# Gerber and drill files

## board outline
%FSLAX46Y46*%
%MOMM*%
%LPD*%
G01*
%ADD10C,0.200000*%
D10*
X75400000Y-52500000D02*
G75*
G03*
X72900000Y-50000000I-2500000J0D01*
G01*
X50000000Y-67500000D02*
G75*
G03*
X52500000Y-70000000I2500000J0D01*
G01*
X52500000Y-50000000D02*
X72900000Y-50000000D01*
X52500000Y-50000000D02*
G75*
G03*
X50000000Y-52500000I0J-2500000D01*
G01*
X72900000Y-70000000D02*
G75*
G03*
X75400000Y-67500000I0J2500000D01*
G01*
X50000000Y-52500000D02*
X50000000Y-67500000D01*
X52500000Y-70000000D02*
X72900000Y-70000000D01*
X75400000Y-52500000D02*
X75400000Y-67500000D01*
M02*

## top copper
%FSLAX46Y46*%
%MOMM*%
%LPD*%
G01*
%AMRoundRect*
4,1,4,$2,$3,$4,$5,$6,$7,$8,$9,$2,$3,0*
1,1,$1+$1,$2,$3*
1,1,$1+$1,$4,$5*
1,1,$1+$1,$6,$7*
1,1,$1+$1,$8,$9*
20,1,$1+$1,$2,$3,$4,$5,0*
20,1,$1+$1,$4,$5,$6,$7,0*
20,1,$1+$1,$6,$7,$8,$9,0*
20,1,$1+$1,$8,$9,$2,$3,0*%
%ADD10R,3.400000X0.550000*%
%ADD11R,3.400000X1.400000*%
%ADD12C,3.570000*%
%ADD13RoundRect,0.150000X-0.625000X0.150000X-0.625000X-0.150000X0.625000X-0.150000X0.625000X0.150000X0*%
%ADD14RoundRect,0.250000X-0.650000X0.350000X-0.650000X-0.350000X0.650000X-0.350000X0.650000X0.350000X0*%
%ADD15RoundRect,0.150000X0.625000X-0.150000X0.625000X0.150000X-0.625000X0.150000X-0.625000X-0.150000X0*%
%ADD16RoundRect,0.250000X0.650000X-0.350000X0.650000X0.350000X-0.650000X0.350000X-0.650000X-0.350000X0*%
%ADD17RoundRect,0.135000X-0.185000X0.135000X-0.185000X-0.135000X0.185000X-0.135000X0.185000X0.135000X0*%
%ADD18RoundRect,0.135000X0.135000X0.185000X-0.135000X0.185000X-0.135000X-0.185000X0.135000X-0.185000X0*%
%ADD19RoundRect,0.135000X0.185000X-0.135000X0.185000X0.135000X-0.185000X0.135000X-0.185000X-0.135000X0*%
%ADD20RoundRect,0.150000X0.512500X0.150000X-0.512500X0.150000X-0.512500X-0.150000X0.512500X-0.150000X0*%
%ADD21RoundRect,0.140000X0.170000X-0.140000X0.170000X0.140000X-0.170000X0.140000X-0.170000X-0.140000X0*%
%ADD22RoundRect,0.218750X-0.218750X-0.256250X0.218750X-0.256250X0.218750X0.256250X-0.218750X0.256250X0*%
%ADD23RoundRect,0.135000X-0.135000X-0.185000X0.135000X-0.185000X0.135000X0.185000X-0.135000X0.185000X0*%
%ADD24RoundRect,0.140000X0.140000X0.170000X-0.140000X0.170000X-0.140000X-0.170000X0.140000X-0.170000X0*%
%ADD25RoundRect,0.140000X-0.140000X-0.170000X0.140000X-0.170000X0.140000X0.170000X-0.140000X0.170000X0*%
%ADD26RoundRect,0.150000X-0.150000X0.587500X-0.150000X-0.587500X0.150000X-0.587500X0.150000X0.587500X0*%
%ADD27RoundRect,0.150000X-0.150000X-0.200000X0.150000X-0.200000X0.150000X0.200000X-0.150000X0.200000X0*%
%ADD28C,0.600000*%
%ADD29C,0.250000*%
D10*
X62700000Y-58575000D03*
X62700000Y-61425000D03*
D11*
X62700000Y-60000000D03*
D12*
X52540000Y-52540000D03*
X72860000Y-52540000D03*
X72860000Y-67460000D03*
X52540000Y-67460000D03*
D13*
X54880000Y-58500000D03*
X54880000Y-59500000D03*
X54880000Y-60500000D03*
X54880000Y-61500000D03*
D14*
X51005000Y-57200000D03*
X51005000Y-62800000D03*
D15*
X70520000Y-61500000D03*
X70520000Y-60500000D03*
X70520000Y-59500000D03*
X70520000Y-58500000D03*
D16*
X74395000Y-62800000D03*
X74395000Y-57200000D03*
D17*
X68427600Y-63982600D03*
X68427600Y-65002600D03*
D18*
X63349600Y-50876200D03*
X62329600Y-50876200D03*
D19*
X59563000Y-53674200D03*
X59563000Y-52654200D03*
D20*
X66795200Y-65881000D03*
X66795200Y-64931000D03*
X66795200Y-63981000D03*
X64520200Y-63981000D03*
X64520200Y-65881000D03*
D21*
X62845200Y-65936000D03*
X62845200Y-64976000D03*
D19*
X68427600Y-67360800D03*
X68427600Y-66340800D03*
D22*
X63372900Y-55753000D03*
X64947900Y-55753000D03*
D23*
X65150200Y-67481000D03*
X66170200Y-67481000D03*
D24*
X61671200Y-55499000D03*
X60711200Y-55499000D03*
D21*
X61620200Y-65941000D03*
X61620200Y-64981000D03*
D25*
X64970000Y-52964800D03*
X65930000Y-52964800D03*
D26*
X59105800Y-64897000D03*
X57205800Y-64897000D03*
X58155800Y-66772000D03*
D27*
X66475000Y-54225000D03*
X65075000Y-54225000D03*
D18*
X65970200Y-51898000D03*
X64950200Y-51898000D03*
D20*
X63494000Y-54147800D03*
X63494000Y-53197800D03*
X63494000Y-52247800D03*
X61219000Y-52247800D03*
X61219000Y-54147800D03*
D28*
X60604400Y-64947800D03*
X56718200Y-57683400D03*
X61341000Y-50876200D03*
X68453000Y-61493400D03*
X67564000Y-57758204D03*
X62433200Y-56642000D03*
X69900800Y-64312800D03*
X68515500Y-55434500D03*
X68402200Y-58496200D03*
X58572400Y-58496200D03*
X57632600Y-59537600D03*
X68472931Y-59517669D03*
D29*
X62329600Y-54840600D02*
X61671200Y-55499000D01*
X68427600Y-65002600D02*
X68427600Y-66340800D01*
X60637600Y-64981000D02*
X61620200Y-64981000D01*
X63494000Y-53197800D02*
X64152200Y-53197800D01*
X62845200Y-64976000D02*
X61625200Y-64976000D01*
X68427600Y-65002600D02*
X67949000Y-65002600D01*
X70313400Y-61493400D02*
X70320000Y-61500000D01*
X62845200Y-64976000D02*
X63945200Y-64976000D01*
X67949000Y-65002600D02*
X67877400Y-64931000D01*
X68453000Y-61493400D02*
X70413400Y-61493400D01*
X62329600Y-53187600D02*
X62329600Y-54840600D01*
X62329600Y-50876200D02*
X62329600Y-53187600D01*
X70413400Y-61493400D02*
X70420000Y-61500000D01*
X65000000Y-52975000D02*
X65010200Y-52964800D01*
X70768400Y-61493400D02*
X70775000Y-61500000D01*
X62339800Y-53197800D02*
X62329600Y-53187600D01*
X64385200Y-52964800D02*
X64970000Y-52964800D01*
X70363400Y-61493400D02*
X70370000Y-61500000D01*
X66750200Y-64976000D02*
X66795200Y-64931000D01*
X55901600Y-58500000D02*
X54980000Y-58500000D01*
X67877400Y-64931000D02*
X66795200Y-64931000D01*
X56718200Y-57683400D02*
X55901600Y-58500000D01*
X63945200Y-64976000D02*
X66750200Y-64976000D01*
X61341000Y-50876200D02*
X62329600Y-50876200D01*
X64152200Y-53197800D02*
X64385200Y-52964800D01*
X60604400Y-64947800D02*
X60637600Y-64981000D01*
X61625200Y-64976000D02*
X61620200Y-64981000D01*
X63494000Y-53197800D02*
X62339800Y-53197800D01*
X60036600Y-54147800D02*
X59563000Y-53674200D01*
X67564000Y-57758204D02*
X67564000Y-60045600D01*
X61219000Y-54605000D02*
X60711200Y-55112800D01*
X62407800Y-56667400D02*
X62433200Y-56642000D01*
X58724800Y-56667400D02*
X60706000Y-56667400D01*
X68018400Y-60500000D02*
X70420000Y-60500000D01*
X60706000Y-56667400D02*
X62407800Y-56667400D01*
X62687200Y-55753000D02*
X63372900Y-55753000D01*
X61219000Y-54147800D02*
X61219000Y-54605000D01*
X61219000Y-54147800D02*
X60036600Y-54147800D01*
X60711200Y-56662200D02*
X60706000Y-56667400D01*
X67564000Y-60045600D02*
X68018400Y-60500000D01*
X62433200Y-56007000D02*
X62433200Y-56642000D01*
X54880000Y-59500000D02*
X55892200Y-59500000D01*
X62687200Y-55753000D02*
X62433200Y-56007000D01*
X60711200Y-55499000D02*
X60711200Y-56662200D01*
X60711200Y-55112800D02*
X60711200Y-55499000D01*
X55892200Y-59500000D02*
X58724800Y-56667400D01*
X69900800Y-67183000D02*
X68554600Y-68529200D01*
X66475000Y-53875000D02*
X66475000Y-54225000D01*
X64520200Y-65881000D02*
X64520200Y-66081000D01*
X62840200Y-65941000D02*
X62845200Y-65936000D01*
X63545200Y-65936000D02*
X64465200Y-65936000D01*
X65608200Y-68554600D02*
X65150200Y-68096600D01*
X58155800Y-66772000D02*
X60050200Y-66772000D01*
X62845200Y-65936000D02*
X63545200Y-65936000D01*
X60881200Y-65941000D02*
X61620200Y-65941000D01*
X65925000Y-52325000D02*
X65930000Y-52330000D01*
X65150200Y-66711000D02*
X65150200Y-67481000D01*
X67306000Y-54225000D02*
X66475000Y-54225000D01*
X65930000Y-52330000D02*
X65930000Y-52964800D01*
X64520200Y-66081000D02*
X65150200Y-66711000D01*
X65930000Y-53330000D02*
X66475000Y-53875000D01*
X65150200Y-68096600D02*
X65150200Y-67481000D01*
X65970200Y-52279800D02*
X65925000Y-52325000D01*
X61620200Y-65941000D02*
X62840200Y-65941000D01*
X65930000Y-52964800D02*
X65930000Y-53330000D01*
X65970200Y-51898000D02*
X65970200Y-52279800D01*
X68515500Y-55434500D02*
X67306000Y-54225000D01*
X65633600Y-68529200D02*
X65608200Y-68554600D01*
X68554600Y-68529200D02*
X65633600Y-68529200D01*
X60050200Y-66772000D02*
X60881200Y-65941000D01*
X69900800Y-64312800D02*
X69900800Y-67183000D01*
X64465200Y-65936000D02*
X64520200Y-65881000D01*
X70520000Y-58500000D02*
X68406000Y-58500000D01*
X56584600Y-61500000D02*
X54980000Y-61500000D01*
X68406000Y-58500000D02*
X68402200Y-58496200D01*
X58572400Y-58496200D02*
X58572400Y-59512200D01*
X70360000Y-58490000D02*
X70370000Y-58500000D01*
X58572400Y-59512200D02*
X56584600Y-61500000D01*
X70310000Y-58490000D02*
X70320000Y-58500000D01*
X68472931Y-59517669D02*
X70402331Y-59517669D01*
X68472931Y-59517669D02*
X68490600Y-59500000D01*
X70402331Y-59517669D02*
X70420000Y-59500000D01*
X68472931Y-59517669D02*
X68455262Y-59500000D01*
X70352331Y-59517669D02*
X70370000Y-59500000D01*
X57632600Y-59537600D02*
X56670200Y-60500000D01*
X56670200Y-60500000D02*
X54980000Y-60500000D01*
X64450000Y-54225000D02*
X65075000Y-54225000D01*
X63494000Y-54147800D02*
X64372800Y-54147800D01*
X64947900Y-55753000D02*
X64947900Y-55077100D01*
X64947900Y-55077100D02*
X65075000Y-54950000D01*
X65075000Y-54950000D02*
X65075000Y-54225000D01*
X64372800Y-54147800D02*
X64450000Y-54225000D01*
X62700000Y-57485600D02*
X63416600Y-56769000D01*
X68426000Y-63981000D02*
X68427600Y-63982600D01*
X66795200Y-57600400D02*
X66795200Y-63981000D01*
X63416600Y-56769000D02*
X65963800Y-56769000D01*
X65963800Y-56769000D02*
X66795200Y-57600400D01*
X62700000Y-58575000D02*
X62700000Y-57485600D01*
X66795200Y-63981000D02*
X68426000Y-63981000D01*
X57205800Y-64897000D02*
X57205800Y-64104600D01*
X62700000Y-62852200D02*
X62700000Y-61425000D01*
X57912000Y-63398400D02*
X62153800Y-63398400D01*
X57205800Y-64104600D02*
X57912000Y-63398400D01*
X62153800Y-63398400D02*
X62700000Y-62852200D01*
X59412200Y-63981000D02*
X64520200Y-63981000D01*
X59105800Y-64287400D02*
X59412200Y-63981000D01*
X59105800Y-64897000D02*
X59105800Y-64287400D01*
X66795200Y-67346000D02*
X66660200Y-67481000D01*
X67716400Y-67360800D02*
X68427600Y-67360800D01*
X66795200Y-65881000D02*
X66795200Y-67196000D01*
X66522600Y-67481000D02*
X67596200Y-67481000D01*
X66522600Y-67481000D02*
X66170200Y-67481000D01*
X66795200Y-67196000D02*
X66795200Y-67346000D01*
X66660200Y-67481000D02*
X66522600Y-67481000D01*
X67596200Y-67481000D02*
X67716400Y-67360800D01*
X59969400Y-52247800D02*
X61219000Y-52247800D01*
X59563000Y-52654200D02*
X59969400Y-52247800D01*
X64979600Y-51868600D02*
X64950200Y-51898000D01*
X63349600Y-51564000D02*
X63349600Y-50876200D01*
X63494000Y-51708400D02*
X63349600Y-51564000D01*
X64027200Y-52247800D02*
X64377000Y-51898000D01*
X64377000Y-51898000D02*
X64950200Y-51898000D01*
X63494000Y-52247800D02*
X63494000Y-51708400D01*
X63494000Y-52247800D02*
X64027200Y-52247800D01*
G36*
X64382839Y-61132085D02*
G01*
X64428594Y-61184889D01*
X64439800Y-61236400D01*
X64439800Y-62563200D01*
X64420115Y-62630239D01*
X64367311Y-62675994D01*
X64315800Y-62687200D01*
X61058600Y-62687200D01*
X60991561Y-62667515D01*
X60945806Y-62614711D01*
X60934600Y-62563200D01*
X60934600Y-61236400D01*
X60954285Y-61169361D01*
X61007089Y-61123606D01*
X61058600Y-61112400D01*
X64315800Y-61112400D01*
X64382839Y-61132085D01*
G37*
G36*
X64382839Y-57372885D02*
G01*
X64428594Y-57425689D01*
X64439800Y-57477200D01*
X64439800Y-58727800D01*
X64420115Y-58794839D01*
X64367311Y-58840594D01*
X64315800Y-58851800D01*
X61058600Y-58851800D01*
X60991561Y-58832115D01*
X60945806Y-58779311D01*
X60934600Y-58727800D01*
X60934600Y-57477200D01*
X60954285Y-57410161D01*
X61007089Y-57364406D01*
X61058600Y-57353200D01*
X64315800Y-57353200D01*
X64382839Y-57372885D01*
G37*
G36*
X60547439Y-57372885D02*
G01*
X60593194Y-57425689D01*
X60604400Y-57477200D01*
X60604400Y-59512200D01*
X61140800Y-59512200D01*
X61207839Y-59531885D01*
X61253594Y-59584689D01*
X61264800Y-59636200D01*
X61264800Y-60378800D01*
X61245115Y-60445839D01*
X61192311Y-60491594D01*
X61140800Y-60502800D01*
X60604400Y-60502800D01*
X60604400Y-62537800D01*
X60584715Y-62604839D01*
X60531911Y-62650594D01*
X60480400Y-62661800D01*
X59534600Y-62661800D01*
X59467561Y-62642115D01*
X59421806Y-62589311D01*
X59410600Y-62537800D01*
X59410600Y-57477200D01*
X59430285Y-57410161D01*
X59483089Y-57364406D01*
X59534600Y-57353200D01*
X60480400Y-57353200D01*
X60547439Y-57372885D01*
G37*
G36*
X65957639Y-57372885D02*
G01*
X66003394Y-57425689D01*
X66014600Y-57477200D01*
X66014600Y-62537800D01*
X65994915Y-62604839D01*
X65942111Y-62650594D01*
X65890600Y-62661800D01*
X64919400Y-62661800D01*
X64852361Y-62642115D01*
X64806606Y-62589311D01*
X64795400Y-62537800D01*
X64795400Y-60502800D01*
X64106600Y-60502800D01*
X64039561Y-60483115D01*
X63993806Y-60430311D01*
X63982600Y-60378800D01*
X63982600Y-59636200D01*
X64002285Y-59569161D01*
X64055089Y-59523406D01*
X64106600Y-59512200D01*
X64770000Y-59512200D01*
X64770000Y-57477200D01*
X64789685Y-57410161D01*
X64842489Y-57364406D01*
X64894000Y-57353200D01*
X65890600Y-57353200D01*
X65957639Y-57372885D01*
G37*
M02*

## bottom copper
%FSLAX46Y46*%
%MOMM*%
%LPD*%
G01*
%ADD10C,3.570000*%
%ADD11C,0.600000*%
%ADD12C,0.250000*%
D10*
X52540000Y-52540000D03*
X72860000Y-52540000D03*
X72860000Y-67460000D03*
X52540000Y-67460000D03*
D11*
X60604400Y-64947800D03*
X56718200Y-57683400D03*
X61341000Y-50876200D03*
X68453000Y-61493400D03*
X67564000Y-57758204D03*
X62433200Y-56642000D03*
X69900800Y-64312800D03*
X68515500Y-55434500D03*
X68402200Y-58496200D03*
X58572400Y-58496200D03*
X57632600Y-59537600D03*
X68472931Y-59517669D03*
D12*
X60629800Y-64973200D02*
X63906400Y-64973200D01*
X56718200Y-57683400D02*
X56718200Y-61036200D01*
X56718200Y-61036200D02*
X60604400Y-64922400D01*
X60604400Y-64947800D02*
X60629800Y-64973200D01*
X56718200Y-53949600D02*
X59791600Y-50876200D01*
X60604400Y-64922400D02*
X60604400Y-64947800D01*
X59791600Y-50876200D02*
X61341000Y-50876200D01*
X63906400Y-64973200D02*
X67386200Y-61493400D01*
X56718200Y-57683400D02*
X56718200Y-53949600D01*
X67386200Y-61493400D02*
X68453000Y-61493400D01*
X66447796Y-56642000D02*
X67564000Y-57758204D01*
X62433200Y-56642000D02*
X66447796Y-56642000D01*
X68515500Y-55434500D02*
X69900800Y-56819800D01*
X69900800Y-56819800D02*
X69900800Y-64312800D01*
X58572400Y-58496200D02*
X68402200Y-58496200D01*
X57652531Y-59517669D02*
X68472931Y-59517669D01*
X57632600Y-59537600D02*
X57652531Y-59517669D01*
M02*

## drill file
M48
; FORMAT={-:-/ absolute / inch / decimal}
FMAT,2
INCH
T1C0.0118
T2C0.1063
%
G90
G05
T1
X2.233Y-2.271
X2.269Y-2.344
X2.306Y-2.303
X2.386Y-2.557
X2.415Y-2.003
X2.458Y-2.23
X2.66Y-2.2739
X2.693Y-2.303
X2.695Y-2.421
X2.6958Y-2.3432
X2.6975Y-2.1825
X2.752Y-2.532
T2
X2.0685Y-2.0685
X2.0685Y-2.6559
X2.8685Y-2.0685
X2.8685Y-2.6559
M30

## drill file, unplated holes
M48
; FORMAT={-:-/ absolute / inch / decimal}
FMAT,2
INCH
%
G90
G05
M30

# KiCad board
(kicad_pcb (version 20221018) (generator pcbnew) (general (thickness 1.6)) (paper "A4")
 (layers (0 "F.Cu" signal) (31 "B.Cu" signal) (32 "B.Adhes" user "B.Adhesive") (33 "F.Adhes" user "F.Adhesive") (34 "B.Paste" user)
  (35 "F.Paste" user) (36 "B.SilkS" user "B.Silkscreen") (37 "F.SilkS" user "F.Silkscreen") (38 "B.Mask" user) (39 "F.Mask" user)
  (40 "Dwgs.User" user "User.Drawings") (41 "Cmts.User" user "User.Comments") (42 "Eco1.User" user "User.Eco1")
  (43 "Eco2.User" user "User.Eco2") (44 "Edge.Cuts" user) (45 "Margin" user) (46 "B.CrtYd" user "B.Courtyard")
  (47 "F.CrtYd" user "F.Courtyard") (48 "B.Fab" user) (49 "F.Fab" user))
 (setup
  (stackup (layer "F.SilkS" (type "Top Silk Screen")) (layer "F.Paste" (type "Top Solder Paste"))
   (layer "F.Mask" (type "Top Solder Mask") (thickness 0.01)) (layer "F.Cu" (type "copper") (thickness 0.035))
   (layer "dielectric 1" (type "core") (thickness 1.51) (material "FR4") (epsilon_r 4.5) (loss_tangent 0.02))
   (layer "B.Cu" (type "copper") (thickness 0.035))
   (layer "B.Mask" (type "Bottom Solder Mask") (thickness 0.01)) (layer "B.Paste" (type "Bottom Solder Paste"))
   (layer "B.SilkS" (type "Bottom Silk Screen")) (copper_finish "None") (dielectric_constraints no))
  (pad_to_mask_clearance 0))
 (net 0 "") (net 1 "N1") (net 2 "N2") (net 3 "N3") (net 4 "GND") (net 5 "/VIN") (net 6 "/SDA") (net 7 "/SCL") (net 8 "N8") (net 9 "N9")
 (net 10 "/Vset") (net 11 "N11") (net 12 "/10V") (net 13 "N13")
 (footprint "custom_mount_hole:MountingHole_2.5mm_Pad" (layer "F.Cu") (at 52.54 52.54)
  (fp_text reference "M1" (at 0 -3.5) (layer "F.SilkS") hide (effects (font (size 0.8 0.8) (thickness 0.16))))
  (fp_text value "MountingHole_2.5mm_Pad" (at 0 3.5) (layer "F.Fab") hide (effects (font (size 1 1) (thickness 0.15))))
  (pad "~" thru_hole circle (at 0 0) (size 3.57 3.57) (drill 2.7) (layers "*.Cu" "*.Mask")))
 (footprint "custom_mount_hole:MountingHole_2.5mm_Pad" (layer "F.Cu") (at 72.86 52.54)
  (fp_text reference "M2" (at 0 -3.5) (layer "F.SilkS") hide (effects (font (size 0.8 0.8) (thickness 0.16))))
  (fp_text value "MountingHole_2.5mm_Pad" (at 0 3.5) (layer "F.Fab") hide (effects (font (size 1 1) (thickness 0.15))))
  (pad "~" thru_hole circle (at 0 0) (size 3.57 3.57) (drill 2.7) (layers "*.Cu" "*.Mask")))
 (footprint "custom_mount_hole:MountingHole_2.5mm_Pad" (layer "F.Cu") (at 72.86 67.46)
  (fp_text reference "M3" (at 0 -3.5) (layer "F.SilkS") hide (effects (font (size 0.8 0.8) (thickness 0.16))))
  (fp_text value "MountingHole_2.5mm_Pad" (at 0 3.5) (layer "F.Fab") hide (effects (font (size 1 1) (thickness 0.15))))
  (pad "~" thru_hole circle (at 0 0) (size 3.57 3.57) (drill 2.7) (layers "*.Cu" "*.Mask")))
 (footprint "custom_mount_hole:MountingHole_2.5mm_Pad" (layer "F.Cu") (at 52.54 67.46)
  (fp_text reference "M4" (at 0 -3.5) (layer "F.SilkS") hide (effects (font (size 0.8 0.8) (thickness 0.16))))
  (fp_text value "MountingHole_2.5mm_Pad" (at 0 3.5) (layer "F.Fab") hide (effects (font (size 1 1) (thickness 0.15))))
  (pad "~" thru_hole circle (at 0 0) (size 3.57 3.57) (drill 2.7) (layers "*.Cu" "*.Mask")))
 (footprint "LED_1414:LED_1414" (layer "F.Cu") (at 62.7 60 -90)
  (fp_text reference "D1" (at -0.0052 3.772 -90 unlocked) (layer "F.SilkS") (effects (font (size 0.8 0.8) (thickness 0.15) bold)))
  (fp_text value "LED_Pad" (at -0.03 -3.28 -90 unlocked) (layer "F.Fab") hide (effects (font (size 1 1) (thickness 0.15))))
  (pad "1" smd rect (at -1.425 0 270) (size 0.55 3.4) (layers "F.Cu" "F.Paste" "F.Mask") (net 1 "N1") (thermal_bridge_angle 45))
  (pad "2" smd rect (at 1.425 0 270) (size 0.55 3.4) (layers "F.Cu" "F.Paste" "F.Mask") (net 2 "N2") (thermal_bridge_angle 45))
  (pad "3" smd rect (at 0 0 270) (size 1.4 3.4) (layers "F.Cu" "F.Paste" "F.Mask") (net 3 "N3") (thermal_bridge_angle 45)))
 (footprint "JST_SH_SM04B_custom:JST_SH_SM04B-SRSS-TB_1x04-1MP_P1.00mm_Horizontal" (layer "F.Cu") (at 52.88 60 -90)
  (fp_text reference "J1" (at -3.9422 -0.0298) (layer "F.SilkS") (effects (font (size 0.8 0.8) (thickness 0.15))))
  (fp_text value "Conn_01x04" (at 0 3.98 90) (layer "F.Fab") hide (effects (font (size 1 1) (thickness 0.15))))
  (pad "1" smd roundrect (at -1.5 -2 270) (size 0.6 1.55) (layers "F.Cu" "F.Paste" "F.Mask") (roundrect_rratio 0.25) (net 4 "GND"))
  (pad "2" smd roundrect (at -0.5 -2 270) (size 0.6 1.55) (layers "F.Cu" "F.Paste" "F.Mask") (roundrect_rratio 0.25) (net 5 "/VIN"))
  (pad "3" smd roundrect (at 0.5 -2 270) (size 0.6 1.55) (layers "F.Cu" "F.Paste" "F.Mask") (roundrect_rratio 0.25) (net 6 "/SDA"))
  (pad "4" smd roundrect (at 1.5 -2 270) (size 0.6 1.55) (layers "F.Cu" "F.Paste" "F.Mask") (roundrect_rratio 0.25) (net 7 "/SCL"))
  (pad "MP" smd roundrect (at -2.8 1.875 270) (size 1.2 1.8) (layers "F.Cu" "F.Paste" "F.Mask") (roundrect_rratio 0.2083333333))
  (pad "MP" smd roundrect (at 2.8 1.875 270) (size 1.2 1.8) (layers "F.Cu" "F.Paste" "F.Mask") (roundrect_rratio 0.2083333333)))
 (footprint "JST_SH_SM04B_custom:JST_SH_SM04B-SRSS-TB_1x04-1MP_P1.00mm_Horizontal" (layer "F.Cu") (at 72.52 60 90)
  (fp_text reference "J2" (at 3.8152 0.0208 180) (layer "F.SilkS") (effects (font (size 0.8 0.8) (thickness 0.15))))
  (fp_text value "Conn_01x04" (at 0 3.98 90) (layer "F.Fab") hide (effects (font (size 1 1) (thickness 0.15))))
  (pad "1" smd roundrect (at -1.5 -2 90) (size 0.6 1.55) (layers "F.Cu" "F.Paste" "F.Mask") (roundrect_rratio 0.25) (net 4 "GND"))
  (pad "2" smd roundrect (at -0.5 -2 90) (size 0.6 1.55) (layers "F.Cu" "F.Paste" "F.Mask") (roundrect_rratio 0.25) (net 5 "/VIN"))
  (pad "3" smd roundrect (at 0.5 -2 90) (size 0.6 1.55) (layers "F.Cu" "F.Paste" "F.Mask") (roundrect_rratio 0.25) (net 6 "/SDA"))
  (pad "4" smd roundrect (at 1.5 -2 90) (size 0.6 1.55) (layers "F.Cu" "F.Paste" "F.Mask") (roundrect_rratio 0.25) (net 7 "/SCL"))
  (pad "MP" smd roundrect (at -2.8 1.875 90) (size 1.2 1.8) (layers "F.Cu" "F.Paste" "F.Mask") (roundrect_rratio 0.2083333333))
  (pad "MP" smd roundrect (at 2.8 1.875 90) (size 1.2 1.8) (layers "F.Cu" "F.Paste" "F.Mask") (roundrect_rratio 0.2083333333)))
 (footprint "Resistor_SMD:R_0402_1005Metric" (layer "F.Cu") (at 68.4276 64.4926 -90)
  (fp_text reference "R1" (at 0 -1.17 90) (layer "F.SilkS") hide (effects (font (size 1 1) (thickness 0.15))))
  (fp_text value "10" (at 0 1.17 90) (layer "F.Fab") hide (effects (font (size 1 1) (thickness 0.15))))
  (pad "1" smd roundrect (at -0.51 0 270) (size 0.54 0.64) (layers "F.Cu" "F.Paste" "F.Mask") (roundrect_rratio 0.25) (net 1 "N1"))
  (pad "2" smd roundrect (at 0.51 0 270) (size 0.54 0.64) (layers "F.Cu" "F.Paste" "F.Mask") (roundrect_rratio 0.25) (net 4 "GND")))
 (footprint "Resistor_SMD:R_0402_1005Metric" (layer "F.Cu") (at 62.8396 50.8762 180)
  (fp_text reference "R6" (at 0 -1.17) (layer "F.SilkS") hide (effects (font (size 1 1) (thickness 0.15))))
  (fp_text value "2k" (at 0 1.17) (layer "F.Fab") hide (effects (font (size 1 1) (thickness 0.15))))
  (pad "1" smd roundrect (at -0.51 0 180) (size 0.54 0.64) (layers "F.Cu" "F.Paste" "F.Mask") (roundrect_rratio 0.25) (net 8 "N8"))
  (pad "2" smd roundrect (at 0.51 0 180) (size 0.54 0.64) (layers "F.Cu" "F.Paste" "F.Mask") (roundrect_rratio 0.25) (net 4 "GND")))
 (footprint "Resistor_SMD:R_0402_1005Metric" (layer "F.Cu") (at 59.563 53.1642 90)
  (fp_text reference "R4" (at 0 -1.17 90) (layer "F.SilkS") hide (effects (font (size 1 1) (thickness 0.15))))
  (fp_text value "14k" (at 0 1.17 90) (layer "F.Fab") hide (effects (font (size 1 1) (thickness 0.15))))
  (pad "1" smd roundrect (at -0.51 0 90) (size 0.54 0.64) (layers "F.Cu" "F.Paste" "F.Mask") (roundrect_rratio 0.25) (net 5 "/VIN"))
  (pad "2" smd roundrect (at 0.51 0 90) (size 0.54 0.64) (layers "F.Cu" "F.Paste" "F.Mask") (roundrect_rratio 0.25) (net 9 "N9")))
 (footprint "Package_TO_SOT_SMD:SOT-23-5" (layer "F.Cu") (at 65.6577 64.931 180)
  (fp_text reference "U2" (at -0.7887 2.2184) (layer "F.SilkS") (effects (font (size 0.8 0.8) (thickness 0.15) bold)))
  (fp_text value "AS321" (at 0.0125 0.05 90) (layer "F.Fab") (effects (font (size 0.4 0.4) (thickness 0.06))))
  (pad "1" smd roundrect (at -1.1375 -0.95 180) (size 1.325 0.6) (layers "F.Cu" "F.Paste" "F.Mask") (roundrect_rratio 0.25) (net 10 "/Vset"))
  (pad "2" smd roundrect (at -1.1375 0 180) (size 1.325 0.6) (layers "F.Cu" "F.Paste" "F.Mask") (roundrect_rratio 0.25) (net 4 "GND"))
  (pad "3" smd roundrect (at -1.1375 0.95 180) (size 1.325 0.6) (layers "F.Cu" "F.Paste" "F.Mask") (roundrect_rratio 0.25) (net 1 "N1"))
  (pad "4" smd roundrect (at 1.1375 0.95 180) (size 1.325 0.6) (layers "F.Cu" "F.Paste" "F.Mask") (roundrect_rratio 0.25) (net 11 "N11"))
  (pad "5" smd roundrect (at 1.1375 -0.95 180) (size 1.325 0.6) (layers "F.Cu" "F.Paste" "F.Mask") (roundrect_rratio 0.25) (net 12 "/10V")))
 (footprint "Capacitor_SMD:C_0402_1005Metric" (layer "F.Cu") (at 62.8452 65.456 90)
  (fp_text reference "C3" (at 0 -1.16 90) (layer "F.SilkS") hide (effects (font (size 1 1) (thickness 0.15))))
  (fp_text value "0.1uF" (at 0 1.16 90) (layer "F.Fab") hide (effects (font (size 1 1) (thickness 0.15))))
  (pad "1" smd roundrect (at -0.48 0 90) (size 0.56 0.62) (layers "F.Cu" "F.Paste" "F.Mask") (roundrect_rratio 0.25) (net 12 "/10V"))
  (pad "2" smd roundrect (at 0.48 0 90) (size 0.56 0.62) (layers "F.Cu" "F.Paste" "F.Mask") (roundrect_rratio 0.25) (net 4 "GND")))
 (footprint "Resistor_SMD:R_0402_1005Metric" (layer "F.Cu") (at 68.4276 66.8508 90)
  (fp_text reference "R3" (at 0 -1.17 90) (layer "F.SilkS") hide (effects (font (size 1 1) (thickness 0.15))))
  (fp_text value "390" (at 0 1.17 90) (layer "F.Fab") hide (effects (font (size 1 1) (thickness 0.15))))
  (pad "1" smd roundrect (at -0.51 0 90) (size 0.54 0.64) (layers "F.Cu" "F.Paste" "F.Mask") (roundrect_rratio 0.25) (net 10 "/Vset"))
  (pad "2" smd roundrect (at 0.51 0 90) (size 0.54 0.64) (layers "F.Cu" "F.Paste" "F.Mask") (roundrect_rratio 0.25) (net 4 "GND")))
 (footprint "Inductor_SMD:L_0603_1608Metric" (layer "F.Cu") (at 64.1604 55.753)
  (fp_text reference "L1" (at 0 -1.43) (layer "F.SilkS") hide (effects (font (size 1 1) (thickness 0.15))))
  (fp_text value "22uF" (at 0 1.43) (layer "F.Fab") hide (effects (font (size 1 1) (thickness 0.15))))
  (pad "1" smd roundrect (at -0.7875 0) (size 0.875 0.95) (layers "F.Cu" "F.Paste" "F.Mask") (roundrect_rratio 0.25) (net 5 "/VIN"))
  (pad "2" smd roundrect (at 0.7875 0) (size 0.875 0.95) (layers "F.Cu" "F.Paste" "F.Mask") (roundrect_rratio 0.25) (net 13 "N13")))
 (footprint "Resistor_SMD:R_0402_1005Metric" (layer "F.Cu") (at 65.6602 67.481)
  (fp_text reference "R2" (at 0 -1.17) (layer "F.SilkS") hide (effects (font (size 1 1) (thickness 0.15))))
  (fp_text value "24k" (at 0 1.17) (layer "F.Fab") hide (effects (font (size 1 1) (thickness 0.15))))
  (pad "1" smd roundrect (at -0.51 0) (size 0.54 0.64) (layers "F.Cu" "F.Paste" "F.Mask") (roundrect_rratio 0.25) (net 12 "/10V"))
  (pad "2" smd roundrect (at 0.51 0) (size 0.54 0.64) (layers "F.Cu" "F.Paste" "F.Mask") (roundrect_rratio 0.25) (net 10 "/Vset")))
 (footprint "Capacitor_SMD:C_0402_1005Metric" (layer "F.Cu") (at 61.1912 55.499 180)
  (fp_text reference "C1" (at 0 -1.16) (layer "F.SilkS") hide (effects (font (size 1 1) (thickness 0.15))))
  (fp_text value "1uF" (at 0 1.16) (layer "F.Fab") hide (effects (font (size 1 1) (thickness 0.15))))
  (pad "1" smd roundrect (at -0.48 0 180) (size 0.56 0.62) (layers "F.Cu" "F.Paste" "F.Mask") (roundrect_rratio 0.25) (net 4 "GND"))
  (pad "2" smd roundrect (at 0.48 0 180) (size 0.56 0.62) (layers "F.Cu" "F.Paste" "F.Mask") (roundrect_rratio 0.25) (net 5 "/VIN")))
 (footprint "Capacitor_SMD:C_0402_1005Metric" (layer "F.Cu") (at 61.6202 65.461 90)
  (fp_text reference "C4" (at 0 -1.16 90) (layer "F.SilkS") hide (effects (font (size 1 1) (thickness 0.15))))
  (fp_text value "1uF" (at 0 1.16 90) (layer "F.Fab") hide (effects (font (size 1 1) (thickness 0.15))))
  (pad "1" smd roundrect (at -0.48 0 90) (size 0.56 0.62) (layers "F.Cu" "F.Paste" "F.Mask") (roundrect_rratio 0.25) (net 12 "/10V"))
  (pad "2" smd roundrect (at 0.48 0 90) (size 0.56 0.62) (layers "F.Cu" "F.Paste" "F.Mask") (roundrect_rratio 0.25) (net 4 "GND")))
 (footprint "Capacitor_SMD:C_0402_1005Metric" (layer "F.Cu") (at 65.45 52.9648)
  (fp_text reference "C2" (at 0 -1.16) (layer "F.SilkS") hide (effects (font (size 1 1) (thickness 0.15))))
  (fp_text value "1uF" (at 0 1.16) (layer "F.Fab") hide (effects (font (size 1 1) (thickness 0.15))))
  (pad "1" smd roundrect (at -0.48 0) (size 0.56 0.62) (layers "F.Cu" "F.Paste" "F.Mask") (roundrect_rratio 0.25) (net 4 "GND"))
  (pad "2" smd roundrect (at 0.48 0) (size 0.56 0.62) (layers "F.Cu" "F.Paste" "F.Mask") (roundrect_rratio 0.25) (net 12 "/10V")))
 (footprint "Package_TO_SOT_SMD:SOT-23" (layer "F.Cu") (at 58.1558 65.8345 -90)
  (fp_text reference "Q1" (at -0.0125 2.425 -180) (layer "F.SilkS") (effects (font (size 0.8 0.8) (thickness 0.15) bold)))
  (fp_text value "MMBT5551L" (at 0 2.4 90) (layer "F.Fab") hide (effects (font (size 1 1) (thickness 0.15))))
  (pad "1" smd roundrect (at -0.9375 -0.95 270) (size 1.475 0.6) (layers "F.Cu" "F.Paste" "F.Mask") (roundrect_rratio 0.25) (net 11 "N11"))
  (pad "2" smd roundrect (at -0.9375 0.95 270) (size 1.475 0.6) (layers "F.Cu" "F.Paste" "F.Mask") (roundrect_rratio 0.25) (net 2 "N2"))
  (pad "3" smd roundrect (at 0.9375 0 270) (size 1.475 0.6) (layers "F.Cu" "F.Paste" "F.Mask") (roundrect_rratio 0.25) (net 12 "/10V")))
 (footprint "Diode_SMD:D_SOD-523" (layer "F.Cu") (at 65.775 54.225 180)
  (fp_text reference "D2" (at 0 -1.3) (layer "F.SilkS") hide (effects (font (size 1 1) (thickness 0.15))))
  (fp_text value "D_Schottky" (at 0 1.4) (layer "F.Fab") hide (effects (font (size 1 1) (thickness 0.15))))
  (pad "1" smd roundrect (at -0.7 0) (size 0.6 0.7) (layers "F.Cu" "F.Paste" "F.Mask") (roundrect_rratio 0.25) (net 12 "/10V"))
  (pad "2" smd roundrect (at 0.7 0) (size 0.6 0.7) (layers "F.Cu" "F.Paste" "F.Mask") (roundrect_rratio 0.25) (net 13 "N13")))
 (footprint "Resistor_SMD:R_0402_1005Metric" (layer "F.Cu") (at 65.4602 51.898 180)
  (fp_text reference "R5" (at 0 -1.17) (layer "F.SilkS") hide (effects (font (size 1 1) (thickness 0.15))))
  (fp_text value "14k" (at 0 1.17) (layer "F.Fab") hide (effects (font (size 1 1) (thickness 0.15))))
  (pad "1" smd roundrect (at -0.51 0 180) (size 0.54 0.64) (layers "F.Cu" "F.Paste" "F.Mask") (roundrect_rratio 0.25) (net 12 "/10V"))
  (pad "2" smd roundrect (at 0.51 0 180) (size 0.54 0.64) (layers "F.Cu" "F.Paste" "F.Mask") (roundrect_rratio 0.25) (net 8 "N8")))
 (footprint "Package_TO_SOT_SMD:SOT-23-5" (layer "F.Cu") (at 62.3565 53.1978 180)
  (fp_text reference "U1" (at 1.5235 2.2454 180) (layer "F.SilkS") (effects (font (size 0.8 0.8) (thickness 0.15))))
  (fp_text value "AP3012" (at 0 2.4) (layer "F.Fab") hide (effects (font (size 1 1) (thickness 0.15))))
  (pad "1" smd roundrect (at -1.1375 -0.95 180) (size 1.325 0.6) (layers "F.Cu" "F.Paste" "F.Mask") (roundrect_rratio 0.25) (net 13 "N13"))
  (pad "2" smd roundrect (at -1.1375 0 180) (size 1.325 0.6) (layers "F.Cu" "F.Paste" "F.Mask") (roundrect_rratio 0.25) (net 4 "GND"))
  (pad "3" smd roundrect (at -1.1375 0.95 180) (size 1.325 0.6) (layers "F.Cu" "F.Paste" "F.Mask") (roundrect_rratio 0.25) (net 8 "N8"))
  (pad "4" smd roundrect (at 1.1375 0.95 180) (size 1.325 0.6) (layers "F.Cu" "F.Paste" "F.Mask") (roundrect_rratio 0.25) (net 9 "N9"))
  (pad "5" smd roundrect (at 1.1375 -0.95 180) (size 1.325 0.6) (layers "F.Cu" "F.Paste" "F.Mask") (roundrect_rratio 0.25) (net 5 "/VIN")))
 (gr_arc (start 72.9 50) (mid 74.667767 50.732233) (end 75.4 52.5) (stroke (width 0.2) (type solid)) (layer "Edge.Cuts"))
 (gr_arc (start 52.5 70) (mid 50.732233 69.267767) (end 50 67.5) (stroke (width 0.2) (type solid)) (layer "Edge.Cuts"))
 (gr_line (start 52.5 50) (end 72.9 50) (stroke (width 0.2) (type solid)) (layer "Edge.Cuts"))
 (gr_arc (start 50 52.5) (mid 50.732233 50.732233) (end 52.5 50) (stroke (width 0.2) (type solid)) (layer "Edge.Cuts"))
 (gr_arc (start 75.4 67.5) (mid 74.667767 69.267767) (end 72.9 70) (stroke (width 0.2) (type solid)) (layer "Edge.Cuts"))
 (gr_line (start 50 52.5) (end 50 67.5) (stroke (width 0.2) (type solid)) (layer "Edge.Cuts"))
 (gr_line (start 52.5 70) (end 72.9 70) (stroke (width 0.2) (type solid)) (layer "Edge.Cuts"))
 (gr_line (start 75.4 52.5) (end 75.4 67.5) (stroke (width 0.2) (type solid)) (layer "Edge.Cuts"))
 (segment (start 62.3296 54.8406) (end 61.6712 55.499) (width 0.25) (layer "F.Cu") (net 4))
 (segment (start 68.4276 65.0026) (end 68.4276 66.3408) (width 0.25) (layer "F.Cu") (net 4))
 (segment (start 60.6376 64.981) (end 61.6202 64.981) (width 0.25) (layer "F.Cu") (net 4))
 (segment (start 63.494 53.1978) (end 64.1522 53.1978) (width 0.25) (layer "F.Cu") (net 4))
 (segment (start 62.8452 64.976) (end 61.6252 64.976) (width 0.25) (layer "F.Cu") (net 4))
 (segment (start 68.4276 65.0026) (end 67.949 65.0026) (width 0.25) (layer "F.Cu") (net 4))
 (segment (start 70.3134 61.4934) (end 70.32 61.5) (width 0.25) (layer "F.Cu") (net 4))
 (segment (start 62.8452 64.976) (end 63.9452 64.976) (width 0.25) (layer "F.Cu") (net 4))
 (segment (start 67.949 65.0026) (end 67.8774 64.931) (width 0.25) (layer "F.Cu") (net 4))
 (segment (start 68.453 61.4934) (end 70.4134 61.4934) (width 0.25) (layer "F.Cu") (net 4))
 (segment (start 62.3296 53.1876) (end 62.3296 54.8406) (width 0.25) (layer "F.Cu") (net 4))
 (segment (start 62.3296 50.8762) (end 62.3296 53.1876) (width 0.25) (layer "F.Cu") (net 4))
 (segment (start 70.4134 61.4934) (end 70.42 61.5) (width 0.25) (layer "F.Cu") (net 4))
 (segment (start 65 52.975) (end 65.0102 52.9648) (width 0.25) (layer "F.Cu") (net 4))
 (segment (start 70.7684 61.4934) (end 70.775 61.5) (width 0.25) (layer "F.Cu") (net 4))
 (segment (start 62.3398 53.1978) (end 62.3296 53.1876) (width 0.25) (layer "F.Cu") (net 4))
 (segment (start 64.3852 52.9648) (end 64.97 52.9648) (width 0.25) (layer "F.Cu") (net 4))
 (segment (start 70.3634 61.4934) (end 70.37 61.5) (width 0.25) (layer "F.Cu") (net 4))
 (segment (start 66.7502 64.976) (end 66.7952 64.931) (width 0.25) (layer "F.Cu") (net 4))
 (segment (start 55.9016 58.5) (end 54.98 58.5) (width 0.25) (layer "F.Cu") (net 4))
 (segment (start 67.8774 64.931) (end 66.7952 64.931) (width 0.25) (layer "F.Cu") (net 4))
 (segment (start 56.7182 57.6834) (end 55.9016 58.5) (width 0.25) (layer "F.Cu") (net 4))
 (segment (start 63.9452 64.976) (end 66.7502 64.976) (width 0.25) (layer "F.Cu") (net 4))
 (segment (start 61.341 50.8762) (end 62.3296 50.8762) (width 0.25) (layer "F.Cu") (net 4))
 (segment (start 64.1522 53.1978) (end 64.3852 52.9648) (width 0.25) (layer "F.Cu") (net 4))
 (segment (start 60.6044 64.9478) (end 60.6376 64.981) (width 0.25) (layer "F.Cu") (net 4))
 (segment (start 61.6252 64.976) (end 61.6202 64.981) (width 0.25) (layer "F.Cu") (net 4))
 (segment (start 63.494 53.1978) (end 62.3398 53.1978) (width 0.25) (layer "F.Cu") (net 4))
 (via (at 60.6044 64.9478) (size 0.6) (drill 0.3) (layers "F.Cu" "B.Cu") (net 4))
 (via (at 56.7182 57.6834) (size 0.6) (drill 0.3) (layers "F.Cu" "B.Cu") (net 4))
 (via (at 61.341 50.8762) (size 0.6) (drill 0.3) (layers "F.Cu" "B.Cu") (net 4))
 (via (at 68.453 61.4934) (size 0.6) (drill 0.3) (layers "F.Cu" "B.Cu") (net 4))
 (segment (start 60.6298 64.9732) (end 63.9064 64.9732) (width 0.25) (layer "B.Cu") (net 4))
 (segment (start 56.7182 57.6834) (end 56.7182 61.0362) (width 0.25) (layer "B.Cu") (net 4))
 (segment (start 56.7182 61.0362) (end 60.6044 64.9224) (width 0.25) (layer "B.Cu") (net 4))
 (segment (start 60.6044 64.9478) (end 60.6298 64.9732) (width 0.25) (layer "B.Cu") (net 4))
 (segment (start 56.7182 53.9496) (end 59.7916 50.8762) (width 0.25) (layer "B.Cu") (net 4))
 (segment (start 60.6044 64.9224) (end 60.6044 64.9478) (width 0.25) (layer "B.Cu") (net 4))
 (segment (start 59.7916 50.8762) (end 61.341 50.8762) (width 0.25) (layer "B.Cu") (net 4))
 (segment (start 63.9064 64.9732) (end 67.3862 61.4934) (width 0.25) (layer "B.Cu") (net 4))
 (segment (start 56.7182 57.6834) (end 56.7182 53.9496) (width 0.25) (layer "B.Cu") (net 4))
 (segment (start 67.3862 61.4934) (end 68.453 61.4934) (width 0.25) (layer "B.Cu") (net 4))
 (segment (start 60.0366 54.1478) (end 59.563 53.6742) (width 0.25) (layer "F.Cu") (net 5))
 (segment (start 67.564 57.758204) (end 67.564 60.0456) (width 0.25) (layer "F.Cu") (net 5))
 (segment (start 61.219 54.605) (end 60.7112 55.1128) (width 0.25) (layer "F.Cu") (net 5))
 (segment (start 62.4078 56.6674) (end 62.4332 56.642) (width 0.25) (layer "F.Cu") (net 5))
 (segment (start 58.7248 56.6674) (end 60.706 56.6674) (width 0.25) (layer "F.Cu") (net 5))
 (segment (start 68.0184 60.5) (end 70.42 60.5) (width 0.25) (layer "F.Cu") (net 5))
 (segment (start 60.706 56.6674) (end 62.4078 56.6674) (width 0.25) (layer "F.Cu") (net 5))
 (segment (start 62.6872 55.753) (end 63.3729 55.753) (width 0.25) (layer "F.Cu") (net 5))
 (segment (start 61.219 54.1478) (end 61.219 54.605) (width 0.25) (layer "F.Cu") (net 5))
 (segment (start 61.219 54.1478) (end 60.0366 54.1478) (width 0.25) (layer "F.Cu") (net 5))
 (segment (start 60.7112 56.6622) (end 60.706 56.6674) (width 0.25) (layer "F.Cu") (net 5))
 (segment (start 67.564 60.0456) (end 68.0184 60.5) (width 0.25) (layer "F.Cu") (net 5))
 (segment (start 62.4332 56.007) (end 62.4332 56.642) (width 0.25) (layer "F.Cu") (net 5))
 (segment (start 54.88 59.5) (end 55.8922 59.5) (width 0.25) (layer "F.Cu") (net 5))
 (segment (start 62.6872 55.753) (end 62.4332 56.007) (width 0.25) (layer "F.Cu") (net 5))
 (segment (start 60.7112 55.499) (end 60.7112 56.6622) (width 0.25) (layer "F.Cu") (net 5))
 (segment (start 60.7112 55.1128) (end 60.7112 55.499) (width 0.25) (layer "F.Cu") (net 5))
 (segment (start 55.8922 59.5) (end 58.7248 56.6674) (width 0.25) (layer "F.Cu") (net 5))
 (via (at 67.564 57.758204) (size 0.6) (drill 0.3) (layers "F.Cu" "B.Cu") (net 5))
 (via (at 62.4332 56.642) (size 0.6) (drill 0.3) (layers "F.Cu" "B.Cu") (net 5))
 (segment (start 66.447796 56.642) (end 67.564 57.758204) (width 0.25) (layer "B.Cu") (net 5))
 (segment (start 62.4332 56.642) (end 66.447796 56.642) (width 0.25) (layer "B.Cu") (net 5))
 (segment (start 69.9008 67.183) (end 68.5546 68.5292) (width 0.25) (layer "F.Cu") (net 12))
 (segment (start 66.475 53.875) (end 66.475 54.225) (width 0.25) (layer "F.Cu") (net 12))
 (segment (start 64.5202 65.881) (end 64.5202 66.081) (width 0.25) (layer "F.Cu") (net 12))
 (segment (start 62.8402 65.941) (end 62.8452 65.936) (width 0.25) (layer "F.Cu") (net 12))
 (segment (start 63.5452 65.936) (end 64.4652 65.936) (width 0.25) (layer "F.Cu") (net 12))
 (segment (start 65.6082 68.5546) (end 65.1502 68.0966) (width 0.25) (layer "F.Cu") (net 12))
 (segment (start 58.1558 66.772) (end 60.0502 66.772) (width 0.25) (layer "F.Cu") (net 12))
 (segment (start 62.8452 65.936) (end 63.5452 65.936) (width 0.25) (layer "F.Cu") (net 12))
 (segment (start 60.8812 65.941) (end 61.6202 65.941) (width 0.25) (layer "F.Cu") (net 12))
 (segment (start 65.925 52.325) (end 65.93 52.33) (width 0.25) (layer "F.Cu") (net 12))
 (segment (start 65.1502 66.711) (end 65.1502 67.481) (width 0.25) (layer "F.Cu") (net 12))
 (segment (start 67.306 54.225) (end 66.475 54.225) (width 0.25) (layer "F.Cu") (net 12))
 (segment (start 65.93 52.33) (end 65.93 52.9648) (width 0.25) (layer "F.Cu") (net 12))
 (segment (start 64.5202 66.081) (end 65.1502 66.711) (width 0.25) (layer "F.Cu") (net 12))
 (segment (start 65.93 53.33) (end 66.475 53.875) (width 0.25) (layer "F.Cu") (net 12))
 (segment (start 65.1502 68.0966) (end 65.1502 67.481) (width 0.25) (layer "F.Cu") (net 12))
 (segment (start 65.9702 52.2798) (end 65.925 52.325) (width 0.25) (layer "F.Cu") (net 12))
 (segment (start 61.6202 65.941) (end 62.8402 65.941) (width 0.25) (layer "F.Cu") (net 12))
 (segment (start 65.93 52.9648) (end 65.93 53.33) (width 0.25) (layer "F.Cu") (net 12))
 (segment (start 65.9702 51.898) (end 65.9702 52.2798) (width 0.25) (layer "F.Cu") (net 12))
 (segment (start 68.5155 55.4345) (end 67.306 54.225) (width 0.25) (layer "F.Cu") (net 12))
 (segment (start 65.6336 68.5292) (end 65.6082 68.5546) (width 0.25) (layer "F.Cu") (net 12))
 (segment (start 68.5546 68.5292) (end 65.6336 68.5292) (width 0.25) (layer "F.Cu") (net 12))
 (segment (start 60.0502 66.772) (end 60.8812 65.941) (width 0.25) (layer "F.Cu") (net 12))
 (segment (start 69.9008 64.3128) (end 69.9008 67.183) (width 0.25) (layer "F.Cu") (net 12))
 (segment (start 64.4652 65.936) (end 64.5202 65.881) (width 0.25) (layer "F.Cu") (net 12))
 (via (at 69.9008 64.3128) (size 0.6) (drill 0.3) (layers "F.Cu" "B.Cu") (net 12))
 (via (at 68.5155 55.4345) (size 0.6) (drill 0.3) (layers "F.Cu" "B.Cu") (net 12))
 (segment (start 68.5155 55.4345) (end 69.9008 56.8198) (width 0.25) (layer "B.Cu") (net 12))
 (segment (start 69.9008 56.8198) (end 69.9008 64.3128) (width 0.25) (layer "B.Cu") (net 12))
 (segment (start 70.52 58.5) (end 68.406 58.5) (width 0.25) (layer "F.Cu") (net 7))
 (segment (start 56.5846 61.5) (end 54.98 61.5) (width 0.25) (layer "F.Cu") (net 7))
 (segment (start 68.406 58.5) (end 68.4022 58.4962) (width 0.25) (layer "F.Cu") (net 7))
 (segment (start 58.5724 58.4962) (end 58.5724 59.5122) (width 0.25) (layer "F.Cu") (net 7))
 (segment (start 70.36 58.49) (end 70.37 58.5) (width 0.25) (layer "F.Cu") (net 7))
 (segment (start 58.5724 59.5122) (end 56.5846 61.5) (width 0.25) (layer "F.Cu") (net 7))
 (segment (start 70.31 58.49) (end 70.32 58.5) (width 0.25) (layer "F.Cu") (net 7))
 (via (at 68.4022 58.4962) (size 0.6) (drill 0.3) (layers "F.Cu" "B.Cu") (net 7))
 (via (at 58.5724 58.4962) (size 0.6) (drill 0.3) (layers "F.Cu" "B.Cu") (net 7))
 (segment (start 58.5724 58.4962) (end 68.4022 58.4962) (width 0.25) (layer "B.Cu") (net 7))
 (segment (start 68.472931 59.517669) (end 70.402331 59.517669) (width 0.25) (layer "F.Cu") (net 6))
 (segment (start 68.472931 59.517669) (end 68.4906 59.5) (width 0.25) (layer "F.Cu") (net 6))
 (segment (start 70.402331 59.517669) (end 70.42 59.5) (width 0.25) (layer "F.Cu") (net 6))
 (segment (start 68.472931 59.517669) (end 68.455262 59.5) (width 0.25) (layer "F.Cu") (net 6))
 (segment (start 70.352331 59.517669) (end 70.37 59.5) (width 0.25) (layer "F.Cu") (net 6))
 (segment (start 57.6326 59.5376) (end 56.6702 60.5) (width 0.25) (layer "F.Cu") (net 6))
 (segment (start 56.6702 60.5) (end 54.98 60.5) (width 0.25) (layer "F.Cu") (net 6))
 (via (at 57.6326 59.5376) (size 0.6) (drill 0.3) (layers "F.Cu" "B.Cu") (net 6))
 (via (at 68.472931 59.517669) (size 0.6) (drill 0.3) (layers "F.Cu" "B.Cu") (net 6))
 (segment (start 57.652531 59.517669) (end 68.472931 59.517669) (width 0.25) (layer "B.Cu") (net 6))
 (segment (start 57.6326 59.5376) (end 57.652531 59.517669) (width 0.25) (layer "B.Cu") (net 6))
 (segment (start 64.45 54.225) (end 65.075 54.225) (width 0.25) (layer "F.Cu") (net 13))
 (segment (start 63.494 54.1478) (end 64.3728 54.1478) (width 0.25) (layer "F.Cu") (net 13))
 (segment (start 64.9479 55.753) (end 64.9479 55.0771) (width 0.25) (layer "F.Cu") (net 13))
 (segment (start 64.9479 55.0771) (end 65.075 54.95) (width 0.25) (layer "F.Cu") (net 13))
 (segment (start 65.075 54.95) (end 65.075 54.225) (width 0.25) (layer "F.Cu") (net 13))
 (segment (start 64.3728 54.1478) (end 64.45 54.225) (width 0.25) (layer "F.Cu") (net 13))
 (segment (start 62.7 57.4856) (end 63.4166 56.769) (width 0.25) (layer "F.Cu") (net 1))
 (segment (start 68.426 63.981) (end 68.4276 63.9826) (width 0.25) (layer "F.Cu") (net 1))
 (segment (start 66.7952 57.6004) (end 66.7952 63.981) (width 0.25) (layer "F.Cu") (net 1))
 (segment (start 63.4166 56.769) (end 65.9638 56.769) (width 0.25) (layer "F.Cu") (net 1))
 (segment (start 65.9638 56.769) (end 66.7952 57.6004) (width 0.25) (layer "F.Cu") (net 1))
 (segment (start 62.7 58.575) (end 62.7 57.4856) (width 0.25) (layer "F.Cu") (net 1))
 (segment (start 66.7952 63.981) (end 68.426 63.981) (width 0.25) (layer "F.Cu") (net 1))
 (segment (start 57.2058 64.897) (end 57.2058 64.1046) (width 0.25) (layer "F.Cu") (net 2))
 (segment (start 62.7 62.8522) (end 62.7 61.425) (width 0.25) (layer "F.Cu") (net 2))
 (segment (start 57.912 63.3984) (end 62.1538 63.3984) (width 0.25) (layer "F.Cu") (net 2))
 (segment (start 57.2058 64.1046) (end 57.912 63.3984) (width 0.25) (layer "F.Cu") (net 2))
 (segment (start 62.1538 63.3984) (end 62.7 62.8522) (width 0.25) (layer "F.Cu") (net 2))
 (segment (start 59.4122 63.981) (end 64.5202 63.981) (width 0.25) (layer "F.Cu") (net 11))
 (segment (start 59.1058 64.2874) (end 59.4122 63.981) (width 0.25) (layer "F.Cu") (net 11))
 (segment (start 59.1058 64.897) (end 59.1058 64.2874) (width 0.25) (layer "F.Cu") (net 11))
 (segment (start 66.7952 67.346) (end 66.6602 67.481) (width 0.25) (layer "F.Cu") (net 10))
 (segment (start 67.7164 67.3608) (end 68.4276 67.3608) (width 0.25) (layer "F.Cu") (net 10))
 (segment (start 66.7952 65.881) (end 66.7952 67.196) (width 0.25) (layer "F.Cu") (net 10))
 (segment (start 66.5226 67.481) (end 67.5962 67.481) (width 0.25) (layer "F.Cu") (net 10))
 (segment (start 66.5226 67.481) (end 66.1702 67.481) (width 0.25) (layer "F.Cu") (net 10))
 (segment (start 66.7952 67.196) (end 66.7952 67.346) (width 0.25) (layer "F.Cu") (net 10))
 (segment (start 66.6602 67.481) (end 66.5226 67.481) (width 0.25) (layer "F.Cu") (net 10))
 (segment (start 67.5962 67.481) (end 67.7164 67.3608) (width 0.25) (layer "F.Cu") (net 10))
 (segment (start 59.9694 52.2478) (end 61.219 52.2478) (width 0.25) (layer "F.Cu") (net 9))
 (segment (start 59.563 52.6542) (end 59.9694 52.2478) (width 0.25) (layer "F.Cu") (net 9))
 (segment (start 64.9796 51.8686) (end 64.9502 51.898) (width 0.25) (layer "F.Cu") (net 8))
 (segment (start 63.3496 51.564) (end 63.3496 50.8762) (width 0.25) (layer "F.Cu") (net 8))
 (segment (start 63.494 51.7084) (end 63.3496 51.564) (width 0.25) (layer "F.Cu") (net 8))
 (segment (start 64.0272 52.2478) (end 64.377 51.898) (width 0.25) (layer "F.Cu") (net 8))
 (segment (start 64.377 51.898) (end 64.9502 51.898) (width 0.25) (layer "F.Cu") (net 8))
 (segment (start 63.494 52.2478) (end 63.494 51.7084) (width 0.25) (layer "F.Cu") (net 8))
 (segment (start 63.494 52.2478) (end 64.0272 52.2478) (width 0.25) (layer "F.Cu") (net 8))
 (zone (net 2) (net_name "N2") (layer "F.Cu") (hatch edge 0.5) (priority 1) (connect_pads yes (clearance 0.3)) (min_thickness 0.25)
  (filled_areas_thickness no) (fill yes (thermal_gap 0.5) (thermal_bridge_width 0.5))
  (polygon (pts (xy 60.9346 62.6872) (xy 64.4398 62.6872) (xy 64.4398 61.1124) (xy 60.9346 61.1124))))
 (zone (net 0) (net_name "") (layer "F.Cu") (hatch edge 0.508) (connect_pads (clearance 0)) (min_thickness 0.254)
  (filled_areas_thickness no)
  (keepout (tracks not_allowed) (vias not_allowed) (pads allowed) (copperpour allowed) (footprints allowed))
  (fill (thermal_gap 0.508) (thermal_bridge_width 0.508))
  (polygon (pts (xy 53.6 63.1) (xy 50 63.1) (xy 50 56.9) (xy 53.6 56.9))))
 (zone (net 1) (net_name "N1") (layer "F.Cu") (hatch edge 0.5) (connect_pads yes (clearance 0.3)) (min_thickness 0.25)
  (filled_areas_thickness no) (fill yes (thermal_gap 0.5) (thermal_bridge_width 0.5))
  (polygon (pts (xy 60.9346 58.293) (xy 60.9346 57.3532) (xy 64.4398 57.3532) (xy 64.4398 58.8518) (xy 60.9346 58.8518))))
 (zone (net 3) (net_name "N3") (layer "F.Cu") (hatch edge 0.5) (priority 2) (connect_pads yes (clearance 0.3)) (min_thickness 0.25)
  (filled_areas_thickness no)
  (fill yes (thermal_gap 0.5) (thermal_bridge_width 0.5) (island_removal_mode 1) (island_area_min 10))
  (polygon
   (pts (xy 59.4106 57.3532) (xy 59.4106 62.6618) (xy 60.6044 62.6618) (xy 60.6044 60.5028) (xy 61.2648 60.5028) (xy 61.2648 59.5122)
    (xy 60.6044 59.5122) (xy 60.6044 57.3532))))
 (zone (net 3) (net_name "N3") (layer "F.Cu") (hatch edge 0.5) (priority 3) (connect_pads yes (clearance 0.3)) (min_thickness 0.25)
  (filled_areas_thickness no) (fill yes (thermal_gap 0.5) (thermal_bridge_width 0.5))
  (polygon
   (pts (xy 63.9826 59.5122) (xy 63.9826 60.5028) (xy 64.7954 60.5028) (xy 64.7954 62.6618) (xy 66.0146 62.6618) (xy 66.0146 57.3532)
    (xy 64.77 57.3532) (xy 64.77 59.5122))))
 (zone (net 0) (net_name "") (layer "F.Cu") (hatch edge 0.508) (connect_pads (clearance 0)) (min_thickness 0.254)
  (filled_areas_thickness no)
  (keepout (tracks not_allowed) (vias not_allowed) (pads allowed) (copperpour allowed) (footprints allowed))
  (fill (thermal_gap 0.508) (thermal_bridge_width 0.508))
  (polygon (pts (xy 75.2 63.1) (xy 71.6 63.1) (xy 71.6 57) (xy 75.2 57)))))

